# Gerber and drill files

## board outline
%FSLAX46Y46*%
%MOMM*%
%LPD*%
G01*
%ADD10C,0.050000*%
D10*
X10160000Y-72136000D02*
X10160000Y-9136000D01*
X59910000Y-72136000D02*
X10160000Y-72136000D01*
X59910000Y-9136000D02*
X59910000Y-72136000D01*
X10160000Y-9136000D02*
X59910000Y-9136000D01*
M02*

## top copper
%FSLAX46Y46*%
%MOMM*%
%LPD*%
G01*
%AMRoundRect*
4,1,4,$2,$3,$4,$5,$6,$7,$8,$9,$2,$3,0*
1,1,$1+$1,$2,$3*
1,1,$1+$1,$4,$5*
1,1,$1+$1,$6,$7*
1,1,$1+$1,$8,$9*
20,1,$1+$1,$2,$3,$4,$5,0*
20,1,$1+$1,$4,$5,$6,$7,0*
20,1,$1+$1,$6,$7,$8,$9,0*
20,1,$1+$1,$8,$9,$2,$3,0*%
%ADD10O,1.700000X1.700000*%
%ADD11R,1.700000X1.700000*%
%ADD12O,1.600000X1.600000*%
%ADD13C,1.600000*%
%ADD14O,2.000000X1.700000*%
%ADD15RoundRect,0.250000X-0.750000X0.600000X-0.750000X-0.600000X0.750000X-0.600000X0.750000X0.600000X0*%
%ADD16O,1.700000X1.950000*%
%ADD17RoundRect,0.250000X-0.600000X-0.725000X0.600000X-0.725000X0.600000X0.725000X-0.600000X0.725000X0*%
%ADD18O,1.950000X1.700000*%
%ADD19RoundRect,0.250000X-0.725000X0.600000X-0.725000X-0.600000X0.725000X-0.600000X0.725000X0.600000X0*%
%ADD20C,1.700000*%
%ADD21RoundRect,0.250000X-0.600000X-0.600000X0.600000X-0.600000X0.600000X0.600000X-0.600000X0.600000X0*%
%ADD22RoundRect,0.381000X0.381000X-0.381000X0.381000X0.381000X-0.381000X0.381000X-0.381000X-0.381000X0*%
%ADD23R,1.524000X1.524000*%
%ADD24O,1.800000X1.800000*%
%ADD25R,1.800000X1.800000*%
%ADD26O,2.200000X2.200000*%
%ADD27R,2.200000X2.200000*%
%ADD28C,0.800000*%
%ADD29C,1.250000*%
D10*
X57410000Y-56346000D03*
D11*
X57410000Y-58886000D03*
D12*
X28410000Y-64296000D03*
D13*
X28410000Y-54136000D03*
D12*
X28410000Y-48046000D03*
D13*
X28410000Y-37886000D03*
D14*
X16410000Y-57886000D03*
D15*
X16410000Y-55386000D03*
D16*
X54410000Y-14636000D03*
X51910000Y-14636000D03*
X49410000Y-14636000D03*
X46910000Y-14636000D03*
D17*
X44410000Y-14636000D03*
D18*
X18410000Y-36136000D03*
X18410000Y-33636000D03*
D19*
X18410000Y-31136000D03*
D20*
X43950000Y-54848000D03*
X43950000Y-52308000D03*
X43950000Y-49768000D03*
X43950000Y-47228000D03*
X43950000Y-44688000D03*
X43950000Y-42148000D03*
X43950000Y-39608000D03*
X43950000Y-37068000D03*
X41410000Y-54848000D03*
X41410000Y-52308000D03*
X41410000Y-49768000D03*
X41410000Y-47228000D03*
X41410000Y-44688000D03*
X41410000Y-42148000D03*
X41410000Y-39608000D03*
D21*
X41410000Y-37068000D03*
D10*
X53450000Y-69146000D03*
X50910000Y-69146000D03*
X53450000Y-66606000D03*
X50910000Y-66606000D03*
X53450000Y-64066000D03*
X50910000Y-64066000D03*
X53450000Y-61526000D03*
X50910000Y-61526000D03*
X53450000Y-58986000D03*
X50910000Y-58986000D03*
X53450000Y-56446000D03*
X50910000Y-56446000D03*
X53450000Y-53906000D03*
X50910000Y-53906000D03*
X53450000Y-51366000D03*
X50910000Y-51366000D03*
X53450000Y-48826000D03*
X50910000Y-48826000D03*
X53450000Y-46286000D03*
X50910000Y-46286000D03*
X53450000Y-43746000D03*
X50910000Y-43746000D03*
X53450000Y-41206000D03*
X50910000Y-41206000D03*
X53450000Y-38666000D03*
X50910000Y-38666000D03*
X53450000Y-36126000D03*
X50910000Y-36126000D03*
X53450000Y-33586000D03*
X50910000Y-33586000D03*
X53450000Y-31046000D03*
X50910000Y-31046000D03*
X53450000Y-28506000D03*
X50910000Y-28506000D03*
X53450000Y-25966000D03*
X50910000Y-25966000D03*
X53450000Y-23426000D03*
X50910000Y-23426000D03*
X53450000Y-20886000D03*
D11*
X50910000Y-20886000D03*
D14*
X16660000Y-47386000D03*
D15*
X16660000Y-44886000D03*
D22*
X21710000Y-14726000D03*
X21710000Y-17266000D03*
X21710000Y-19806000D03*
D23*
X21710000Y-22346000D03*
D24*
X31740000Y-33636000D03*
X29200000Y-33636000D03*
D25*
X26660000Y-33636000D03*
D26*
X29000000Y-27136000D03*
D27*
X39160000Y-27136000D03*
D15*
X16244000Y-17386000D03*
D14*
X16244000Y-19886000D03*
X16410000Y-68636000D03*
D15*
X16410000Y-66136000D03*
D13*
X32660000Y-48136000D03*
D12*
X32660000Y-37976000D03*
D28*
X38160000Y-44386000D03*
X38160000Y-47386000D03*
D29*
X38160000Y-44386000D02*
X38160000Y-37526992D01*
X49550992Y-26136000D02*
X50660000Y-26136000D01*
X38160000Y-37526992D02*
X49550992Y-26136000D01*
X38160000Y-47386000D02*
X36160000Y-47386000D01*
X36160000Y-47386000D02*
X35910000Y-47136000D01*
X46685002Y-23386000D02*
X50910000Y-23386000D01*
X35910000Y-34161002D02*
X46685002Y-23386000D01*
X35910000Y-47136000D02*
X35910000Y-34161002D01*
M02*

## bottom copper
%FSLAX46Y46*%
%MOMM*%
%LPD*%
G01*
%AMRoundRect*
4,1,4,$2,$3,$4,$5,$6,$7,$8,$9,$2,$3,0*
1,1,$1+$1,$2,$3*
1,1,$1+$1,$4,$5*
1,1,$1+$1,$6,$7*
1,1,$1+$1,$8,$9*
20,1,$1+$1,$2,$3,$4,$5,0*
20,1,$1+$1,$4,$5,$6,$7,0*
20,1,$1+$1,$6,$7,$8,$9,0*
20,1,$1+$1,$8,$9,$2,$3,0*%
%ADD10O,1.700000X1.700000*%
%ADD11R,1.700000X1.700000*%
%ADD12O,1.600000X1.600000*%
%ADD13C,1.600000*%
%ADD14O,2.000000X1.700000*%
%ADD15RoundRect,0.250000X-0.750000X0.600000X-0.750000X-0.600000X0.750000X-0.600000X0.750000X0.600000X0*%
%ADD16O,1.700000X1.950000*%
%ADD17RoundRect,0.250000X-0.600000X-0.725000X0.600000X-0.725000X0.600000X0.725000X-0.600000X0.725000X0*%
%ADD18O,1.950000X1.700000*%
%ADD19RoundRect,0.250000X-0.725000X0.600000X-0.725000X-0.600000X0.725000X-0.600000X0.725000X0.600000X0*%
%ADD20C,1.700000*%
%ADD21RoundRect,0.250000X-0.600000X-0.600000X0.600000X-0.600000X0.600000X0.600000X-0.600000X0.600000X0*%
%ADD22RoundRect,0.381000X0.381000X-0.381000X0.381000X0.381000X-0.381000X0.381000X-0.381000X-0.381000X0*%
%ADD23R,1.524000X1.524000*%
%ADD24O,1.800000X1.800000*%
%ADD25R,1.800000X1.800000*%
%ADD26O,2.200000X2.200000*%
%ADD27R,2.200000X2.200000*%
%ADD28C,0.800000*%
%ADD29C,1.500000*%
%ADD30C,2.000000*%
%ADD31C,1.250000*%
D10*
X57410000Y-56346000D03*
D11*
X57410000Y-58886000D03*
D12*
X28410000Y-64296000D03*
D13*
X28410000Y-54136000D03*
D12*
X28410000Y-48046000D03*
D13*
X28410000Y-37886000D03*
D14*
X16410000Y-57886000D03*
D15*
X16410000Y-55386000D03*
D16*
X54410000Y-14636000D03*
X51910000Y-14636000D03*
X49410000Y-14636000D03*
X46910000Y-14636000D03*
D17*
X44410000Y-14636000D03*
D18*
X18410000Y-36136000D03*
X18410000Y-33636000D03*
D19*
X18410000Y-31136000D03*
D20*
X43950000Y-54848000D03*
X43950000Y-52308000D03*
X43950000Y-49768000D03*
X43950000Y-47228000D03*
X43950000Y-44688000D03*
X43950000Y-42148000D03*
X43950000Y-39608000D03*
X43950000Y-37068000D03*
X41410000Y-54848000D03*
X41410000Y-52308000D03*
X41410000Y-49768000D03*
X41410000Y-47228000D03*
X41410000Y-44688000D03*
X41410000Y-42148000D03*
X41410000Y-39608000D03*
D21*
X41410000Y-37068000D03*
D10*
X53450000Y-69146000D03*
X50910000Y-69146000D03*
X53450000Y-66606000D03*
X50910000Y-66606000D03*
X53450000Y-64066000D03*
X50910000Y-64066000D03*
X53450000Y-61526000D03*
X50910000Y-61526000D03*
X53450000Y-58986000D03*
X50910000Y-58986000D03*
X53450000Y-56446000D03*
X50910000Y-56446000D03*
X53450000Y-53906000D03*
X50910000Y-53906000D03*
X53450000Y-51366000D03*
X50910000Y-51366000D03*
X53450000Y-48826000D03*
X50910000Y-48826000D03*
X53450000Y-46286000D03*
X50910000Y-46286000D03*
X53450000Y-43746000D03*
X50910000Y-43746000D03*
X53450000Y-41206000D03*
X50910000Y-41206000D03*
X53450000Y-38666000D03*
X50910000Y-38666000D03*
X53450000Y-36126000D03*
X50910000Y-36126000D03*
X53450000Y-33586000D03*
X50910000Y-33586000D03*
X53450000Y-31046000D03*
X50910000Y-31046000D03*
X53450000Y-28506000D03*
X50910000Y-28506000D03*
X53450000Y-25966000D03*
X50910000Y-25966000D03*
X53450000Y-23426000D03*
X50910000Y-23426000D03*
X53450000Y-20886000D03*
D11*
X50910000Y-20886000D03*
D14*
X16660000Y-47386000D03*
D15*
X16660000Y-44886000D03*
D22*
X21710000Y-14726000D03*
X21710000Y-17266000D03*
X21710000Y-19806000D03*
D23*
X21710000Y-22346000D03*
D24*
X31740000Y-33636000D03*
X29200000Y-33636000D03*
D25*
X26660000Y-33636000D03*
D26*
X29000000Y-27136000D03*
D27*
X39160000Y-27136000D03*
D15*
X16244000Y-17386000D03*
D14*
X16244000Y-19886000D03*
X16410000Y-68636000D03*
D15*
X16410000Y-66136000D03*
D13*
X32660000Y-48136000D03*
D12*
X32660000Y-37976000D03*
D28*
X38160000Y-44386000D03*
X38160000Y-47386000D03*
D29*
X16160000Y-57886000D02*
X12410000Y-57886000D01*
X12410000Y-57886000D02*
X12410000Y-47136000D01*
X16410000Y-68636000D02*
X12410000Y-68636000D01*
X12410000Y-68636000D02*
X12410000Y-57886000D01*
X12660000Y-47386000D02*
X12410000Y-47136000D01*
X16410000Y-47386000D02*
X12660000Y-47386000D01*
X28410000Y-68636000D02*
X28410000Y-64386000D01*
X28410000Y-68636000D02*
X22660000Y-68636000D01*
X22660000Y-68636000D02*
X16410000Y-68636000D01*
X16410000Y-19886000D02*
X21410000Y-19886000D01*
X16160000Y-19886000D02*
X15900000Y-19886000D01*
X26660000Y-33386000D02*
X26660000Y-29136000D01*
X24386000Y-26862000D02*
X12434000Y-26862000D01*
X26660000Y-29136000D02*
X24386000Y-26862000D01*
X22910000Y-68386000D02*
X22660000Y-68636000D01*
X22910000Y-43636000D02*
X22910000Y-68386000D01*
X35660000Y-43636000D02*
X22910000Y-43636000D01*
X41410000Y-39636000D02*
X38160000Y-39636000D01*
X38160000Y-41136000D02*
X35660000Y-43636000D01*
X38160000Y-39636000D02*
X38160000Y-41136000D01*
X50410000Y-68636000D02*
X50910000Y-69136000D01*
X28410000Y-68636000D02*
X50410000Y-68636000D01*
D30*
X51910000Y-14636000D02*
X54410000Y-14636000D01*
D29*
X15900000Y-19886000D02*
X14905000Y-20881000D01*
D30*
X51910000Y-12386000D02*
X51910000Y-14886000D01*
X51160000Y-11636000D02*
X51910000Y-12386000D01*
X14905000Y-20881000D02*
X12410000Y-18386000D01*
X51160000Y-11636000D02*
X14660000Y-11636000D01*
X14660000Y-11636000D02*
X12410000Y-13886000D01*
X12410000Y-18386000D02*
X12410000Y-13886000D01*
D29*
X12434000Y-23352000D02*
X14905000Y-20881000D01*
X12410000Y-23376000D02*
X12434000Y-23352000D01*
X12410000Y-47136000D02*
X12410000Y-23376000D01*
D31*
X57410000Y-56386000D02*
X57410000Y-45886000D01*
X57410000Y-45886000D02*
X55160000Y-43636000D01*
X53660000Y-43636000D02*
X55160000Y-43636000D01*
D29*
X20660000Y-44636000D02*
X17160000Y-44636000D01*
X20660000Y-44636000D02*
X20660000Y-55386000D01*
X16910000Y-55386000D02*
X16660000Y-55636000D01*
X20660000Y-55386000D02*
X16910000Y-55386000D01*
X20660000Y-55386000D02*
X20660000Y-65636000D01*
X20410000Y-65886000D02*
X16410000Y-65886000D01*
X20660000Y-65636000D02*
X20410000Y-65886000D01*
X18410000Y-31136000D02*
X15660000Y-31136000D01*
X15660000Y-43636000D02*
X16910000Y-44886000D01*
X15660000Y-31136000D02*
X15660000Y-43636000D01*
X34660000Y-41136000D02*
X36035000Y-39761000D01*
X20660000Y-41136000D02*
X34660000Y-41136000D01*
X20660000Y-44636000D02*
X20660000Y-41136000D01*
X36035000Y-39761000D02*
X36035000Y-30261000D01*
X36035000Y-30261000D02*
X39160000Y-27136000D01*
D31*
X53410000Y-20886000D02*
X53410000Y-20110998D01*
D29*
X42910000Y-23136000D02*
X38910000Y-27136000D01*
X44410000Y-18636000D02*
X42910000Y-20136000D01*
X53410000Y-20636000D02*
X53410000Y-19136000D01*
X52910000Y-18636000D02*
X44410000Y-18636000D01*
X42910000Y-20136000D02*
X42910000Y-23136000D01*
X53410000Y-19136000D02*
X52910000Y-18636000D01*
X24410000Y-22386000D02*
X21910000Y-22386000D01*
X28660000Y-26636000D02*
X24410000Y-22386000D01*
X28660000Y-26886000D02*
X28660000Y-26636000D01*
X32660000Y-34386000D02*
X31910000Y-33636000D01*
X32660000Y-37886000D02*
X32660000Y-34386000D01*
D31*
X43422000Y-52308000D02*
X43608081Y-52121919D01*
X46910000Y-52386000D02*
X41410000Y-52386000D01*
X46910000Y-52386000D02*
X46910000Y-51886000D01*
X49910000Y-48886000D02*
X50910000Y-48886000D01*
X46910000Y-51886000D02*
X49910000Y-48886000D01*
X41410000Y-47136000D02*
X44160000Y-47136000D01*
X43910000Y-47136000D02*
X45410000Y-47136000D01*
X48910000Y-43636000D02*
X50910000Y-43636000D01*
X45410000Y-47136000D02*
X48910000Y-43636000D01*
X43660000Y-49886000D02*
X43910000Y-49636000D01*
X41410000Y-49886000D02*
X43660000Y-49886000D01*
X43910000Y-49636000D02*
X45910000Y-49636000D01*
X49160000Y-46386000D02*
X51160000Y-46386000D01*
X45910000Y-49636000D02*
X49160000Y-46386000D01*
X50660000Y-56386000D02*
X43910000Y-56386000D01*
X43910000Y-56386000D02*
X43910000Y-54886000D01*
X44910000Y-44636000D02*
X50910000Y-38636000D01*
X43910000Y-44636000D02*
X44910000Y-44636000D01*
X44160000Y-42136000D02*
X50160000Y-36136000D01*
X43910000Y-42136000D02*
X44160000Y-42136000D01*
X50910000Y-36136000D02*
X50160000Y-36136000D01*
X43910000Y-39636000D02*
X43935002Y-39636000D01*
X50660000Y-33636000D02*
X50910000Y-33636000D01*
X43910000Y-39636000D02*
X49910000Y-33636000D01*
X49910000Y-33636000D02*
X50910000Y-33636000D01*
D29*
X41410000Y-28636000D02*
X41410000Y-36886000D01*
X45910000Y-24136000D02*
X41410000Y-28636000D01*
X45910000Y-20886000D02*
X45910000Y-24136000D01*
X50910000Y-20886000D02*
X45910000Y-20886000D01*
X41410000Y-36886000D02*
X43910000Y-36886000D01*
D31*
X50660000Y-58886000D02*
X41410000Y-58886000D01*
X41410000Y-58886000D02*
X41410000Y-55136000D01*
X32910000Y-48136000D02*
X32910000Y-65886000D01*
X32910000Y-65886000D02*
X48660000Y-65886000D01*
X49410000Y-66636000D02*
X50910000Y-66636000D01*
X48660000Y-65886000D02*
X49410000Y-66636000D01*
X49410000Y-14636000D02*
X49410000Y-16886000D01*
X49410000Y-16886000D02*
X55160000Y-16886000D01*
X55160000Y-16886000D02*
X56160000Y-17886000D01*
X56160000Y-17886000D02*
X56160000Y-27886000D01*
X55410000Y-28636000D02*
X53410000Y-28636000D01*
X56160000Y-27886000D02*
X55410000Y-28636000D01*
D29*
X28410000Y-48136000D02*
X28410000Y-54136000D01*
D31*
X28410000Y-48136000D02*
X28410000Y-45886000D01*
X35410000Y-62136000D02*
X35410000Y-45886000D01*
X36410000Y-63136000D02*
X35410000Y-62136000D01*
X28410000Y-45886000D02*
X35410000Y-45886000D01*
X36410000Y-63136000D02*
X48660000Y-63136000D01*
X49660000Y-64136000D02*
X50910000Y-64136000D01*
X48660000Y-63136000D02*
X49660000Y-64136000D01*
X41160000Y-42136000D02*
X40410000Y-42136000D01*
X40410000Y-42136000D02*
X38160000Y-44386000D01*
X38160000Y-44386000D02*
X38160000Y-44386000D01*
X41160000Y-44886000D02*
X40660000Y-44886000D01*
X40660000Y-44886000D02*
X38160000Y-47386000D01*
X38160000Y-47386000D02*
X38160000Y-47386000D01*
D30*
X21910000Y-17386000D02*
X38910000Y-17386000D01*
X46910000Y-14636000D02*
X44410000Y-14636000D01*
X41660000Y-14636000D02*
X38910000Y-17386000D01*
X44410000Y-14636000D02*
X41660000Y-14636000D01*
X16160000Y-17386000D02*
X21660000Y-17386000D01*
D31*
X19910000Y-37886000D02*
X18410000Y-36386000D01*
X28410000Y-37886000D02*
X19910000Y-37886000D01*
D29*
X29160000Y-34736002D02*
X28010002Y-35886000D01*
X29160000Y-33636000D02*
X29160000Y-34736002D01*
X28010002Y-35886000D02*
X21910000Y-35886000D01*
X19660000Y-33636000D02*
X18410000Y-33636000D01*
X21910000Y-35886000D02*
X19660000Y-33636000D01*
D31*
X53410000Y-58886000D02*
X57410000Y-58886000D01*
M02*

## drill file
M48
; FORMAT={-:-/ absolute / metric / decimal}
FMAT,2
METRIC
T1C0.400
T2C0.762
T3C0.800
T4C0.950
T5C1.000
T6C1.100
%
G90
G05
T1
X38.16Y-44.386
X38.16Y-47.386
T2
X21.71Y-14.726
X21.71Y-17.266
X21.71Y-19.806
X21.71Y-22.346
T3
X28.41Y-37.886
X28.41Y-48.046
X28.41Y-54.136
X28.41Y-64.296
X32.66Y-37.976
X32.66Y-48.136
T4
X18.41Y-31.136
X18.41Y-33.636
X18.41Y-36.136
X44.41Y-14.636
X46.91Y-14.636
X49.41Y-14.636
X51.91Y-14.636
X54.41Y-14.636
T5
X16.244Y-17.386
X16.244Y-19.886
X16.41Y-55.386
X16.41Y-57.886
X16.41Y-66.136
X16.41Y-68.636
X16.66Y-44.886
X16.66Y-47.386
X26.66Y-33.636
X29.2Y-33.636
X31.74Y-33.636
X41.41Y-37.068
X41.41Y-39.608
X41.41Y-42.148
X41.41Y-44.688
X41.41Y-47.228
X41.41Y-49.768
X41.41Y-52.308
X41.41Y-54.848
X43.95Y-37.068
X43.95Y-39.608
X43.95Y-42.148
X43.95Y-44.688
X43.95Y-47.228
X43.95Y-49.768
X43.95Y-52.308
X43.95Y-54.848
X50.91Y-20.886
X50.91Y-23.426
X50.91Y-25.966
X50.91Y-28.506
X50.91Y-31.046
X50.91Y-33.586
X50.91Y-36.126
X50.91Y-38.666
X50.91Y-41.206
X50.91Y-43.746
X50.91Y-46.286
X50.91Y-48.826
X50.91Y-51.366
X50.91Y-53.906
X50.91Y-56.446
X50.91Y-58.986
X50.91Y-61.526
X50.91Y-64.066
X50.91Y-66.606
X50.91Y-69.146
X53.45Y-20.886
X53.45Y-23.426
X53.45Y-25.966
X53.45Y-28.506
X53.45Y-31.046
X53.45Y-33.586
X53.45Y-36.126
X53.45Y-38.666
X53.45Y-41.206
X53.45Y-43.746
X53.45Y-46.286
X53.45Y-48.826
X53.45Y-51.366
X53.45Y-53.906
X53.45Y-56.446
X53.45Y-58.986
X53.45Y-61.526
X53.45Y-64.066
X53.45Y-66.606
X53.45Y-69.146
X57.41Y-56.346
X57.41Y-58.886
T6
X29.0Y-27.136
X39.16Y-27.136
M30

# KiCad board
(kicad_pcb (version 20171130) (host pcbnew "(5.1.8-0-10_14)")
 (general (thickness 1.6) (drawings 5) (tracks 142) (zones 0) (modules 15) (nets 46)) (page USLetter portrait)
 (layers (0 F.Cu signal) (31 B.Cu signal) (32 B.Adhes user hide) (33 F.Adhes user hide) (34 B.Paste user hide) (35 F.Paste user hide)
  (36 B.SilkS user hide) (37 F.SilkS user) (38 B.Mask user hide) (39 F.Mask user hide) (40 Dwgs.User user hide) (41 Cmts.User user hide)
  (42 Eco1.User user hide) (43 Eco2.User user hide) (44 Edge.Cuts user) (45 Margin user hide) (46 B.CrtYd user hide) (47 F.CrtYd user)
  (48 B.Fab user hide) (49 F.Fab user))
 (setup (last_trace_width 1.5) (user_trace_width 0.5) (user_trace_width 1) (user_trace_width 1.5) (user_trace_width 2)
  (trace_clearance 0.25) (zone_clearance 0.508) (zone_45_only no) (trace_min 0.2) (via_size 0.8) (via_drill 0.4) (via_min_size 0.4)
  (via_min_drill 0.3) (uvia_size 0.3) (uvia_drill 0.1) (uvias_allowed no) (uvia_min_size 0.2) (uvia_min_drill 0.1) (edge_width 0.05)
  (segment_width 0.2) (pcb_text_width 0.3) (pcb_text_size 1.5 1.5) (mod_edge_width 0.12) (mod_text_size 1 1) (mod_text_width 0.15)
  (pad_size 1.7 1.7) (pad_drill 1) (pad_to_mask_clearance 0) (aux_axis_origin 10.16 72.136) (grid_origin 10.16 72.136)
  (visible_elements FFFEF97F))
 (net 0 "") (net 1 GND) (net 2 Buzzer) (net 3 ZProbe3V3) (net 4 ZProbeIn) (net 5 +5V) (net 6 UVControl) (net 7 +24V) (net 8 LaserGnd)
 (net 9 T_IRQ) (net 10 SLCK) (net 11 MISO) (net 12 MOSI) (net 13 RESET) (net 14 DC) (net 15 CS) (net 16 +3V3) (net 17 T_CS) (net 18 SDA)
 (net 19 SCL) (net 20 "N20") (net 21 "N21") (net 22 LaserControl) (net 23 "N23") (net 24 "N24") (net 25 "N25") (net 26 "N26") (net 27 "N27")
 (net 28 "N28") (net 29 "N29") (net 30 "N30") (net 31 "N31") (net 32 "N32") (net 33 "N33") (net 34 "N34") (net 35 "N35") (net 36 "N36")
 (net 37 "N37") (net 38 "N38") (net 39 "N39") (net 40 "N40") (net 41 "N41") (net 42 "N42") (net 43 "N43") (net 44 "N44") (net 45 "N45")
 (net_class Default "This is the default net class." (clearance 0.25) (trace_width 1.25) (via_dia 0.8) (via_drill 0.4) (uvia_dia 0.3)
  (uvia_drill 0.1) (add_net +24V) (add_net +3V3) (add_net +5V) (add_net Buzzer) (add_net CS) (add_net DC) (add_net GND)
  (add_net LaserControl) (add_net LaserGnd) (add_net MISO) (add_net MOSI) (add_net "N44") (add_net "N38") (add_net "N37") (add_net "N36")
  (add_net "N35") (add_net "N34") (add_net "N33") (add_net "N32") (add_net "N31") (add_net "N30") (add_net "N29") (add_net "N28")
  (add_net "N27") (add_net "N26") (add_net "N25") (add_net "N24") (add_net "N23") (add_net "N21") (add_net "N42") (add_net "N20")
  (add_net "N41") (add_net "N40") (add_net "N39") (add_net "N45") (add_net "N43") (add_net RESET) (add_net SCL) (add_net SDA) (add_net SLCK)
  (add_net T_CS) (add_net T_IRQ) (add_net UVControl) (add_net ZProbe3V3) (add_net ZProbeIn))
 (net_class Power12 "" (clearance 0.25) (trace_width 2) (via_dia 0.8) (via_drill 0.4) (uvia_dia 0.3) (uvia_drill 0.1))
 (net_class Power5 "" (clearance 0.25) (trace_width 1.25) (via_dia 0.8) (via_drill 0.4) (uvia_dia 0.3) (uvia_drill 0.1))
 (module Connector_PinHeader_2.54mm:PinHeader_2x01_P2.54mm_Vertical (layer F.Cu) (at 57.41 58.886 90)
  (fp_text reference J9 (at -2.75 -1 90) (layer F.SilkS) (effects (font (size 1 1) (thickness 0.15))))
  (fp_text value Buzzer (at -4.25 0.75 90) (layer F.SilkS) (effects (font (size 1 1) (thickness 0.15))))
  (pad 2 thru_hole oval (at 2.54 0 90) (size 1.7 1.7) (drill 1) (layers *.Cu *.Mask) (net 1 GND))
  (pad 1 thru_hole rect (at 0 0 90) (size 1.7 1.7) (drill 1) (layers *.Cu *.Mask) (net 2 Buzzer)))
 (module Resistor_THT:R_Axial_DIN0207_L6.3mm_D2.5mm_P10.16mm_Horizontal (layer F.Cu) (at 28.41 54.136 270)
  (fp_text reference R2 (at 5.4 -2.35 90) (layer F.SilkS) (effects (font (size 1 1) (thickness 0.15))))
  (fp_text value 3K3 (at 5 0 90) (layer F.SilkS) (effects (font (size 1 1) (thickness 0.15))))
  (pad 2 thru_hole oval (at 10.16 0 270) (size 1.6 1.6) (drill 0.8) (layers *.Cu *.Mask) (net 1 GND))
  (pad 1 thru_hole circle (at 0 0 270) (size 1.6 1.6) (drill 0.8) (layers *.Cu *.Mask) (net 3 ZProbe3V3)))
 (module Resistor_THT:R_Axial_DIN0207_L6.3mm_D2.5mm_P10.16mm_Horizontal (layer F.Cu) (at 28.41 37.886 270)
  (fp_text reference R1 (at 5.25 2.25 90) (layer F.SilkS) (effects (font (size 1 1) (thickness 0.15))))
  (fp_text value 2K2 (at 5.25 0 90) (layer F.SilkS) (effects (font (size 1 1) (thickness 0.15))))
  (pad 2 thru_hole oval (at 10.16 0 270) (size 1.6 1.6) (drill 0.8) (layers *.Cu *.Mask) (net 3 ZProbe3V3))
  (pad 1 thru_hole circle (at 0 0 270) (size 1.6 1.6) (drill 0.8) (layers *.Cu *.Mask) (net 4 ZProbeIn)))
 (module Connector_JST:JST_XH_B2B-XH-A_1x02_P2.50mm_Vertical (layer F.Cu) (at 16.41 55.386 270)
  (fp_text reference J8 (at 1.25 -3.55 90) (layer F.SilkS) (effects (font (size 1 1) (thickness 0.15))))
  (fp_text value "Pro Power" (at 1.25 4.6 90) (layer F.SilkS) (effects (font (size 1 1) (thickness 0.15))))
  (pad 2 thru_hole oval (at 2.5 0 270) (size 1.7 2) (drill 1) (layers *.Cu *.Mask) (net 1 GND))
  (pad 1 thru_hole roundrect (at 0 0 270) (size 1.7 2) (drill 1) (layers *.Cu *.Mask) (roundrect_rratio 0.1470588235294118) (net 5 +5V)))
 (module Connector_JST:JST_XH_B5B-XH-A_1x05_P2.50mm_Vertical (layer F.Cu) (at 44.41 14.636)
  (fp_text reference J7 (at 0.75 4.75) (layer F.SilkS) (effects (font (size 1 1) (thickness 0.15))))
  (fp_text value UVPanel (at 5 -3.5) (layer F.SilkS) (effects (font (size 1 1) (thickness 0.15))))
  (pad 5 thru_hole oval (at 10 0) (size 1.7 1.95) (drill 0.95) (layers *.Cu *.Mask) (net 1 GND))
  (pad 4 thru_hole oval (at 7.5 0) (size 1.7 1.95) (drill 0.95) (layers *.Cu *.Mask) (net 1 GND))
  (pad 3 thru_hole oval (at 5 0) (size 1.7 1.95) (drill 0.95) (layers *.Cu *.Mask) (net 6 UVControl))
  (pad 2 thru_hole oval (at 2.5 0) (size 1.7 1.95) (drill 0.95) (layers *.Cu *.Mask) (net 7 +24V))
  (pad 1 thru_hole roundrect (at 0 0) (size 1.7 1.95) (drill 0.95) (layers *.Cu *.Mask) (roundrect_rratio 0.1470588235294118) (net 7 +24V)))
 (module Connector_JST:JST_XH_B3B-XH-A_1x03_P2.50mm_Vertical (layer F.Cu) (at 18.41 31.136 270)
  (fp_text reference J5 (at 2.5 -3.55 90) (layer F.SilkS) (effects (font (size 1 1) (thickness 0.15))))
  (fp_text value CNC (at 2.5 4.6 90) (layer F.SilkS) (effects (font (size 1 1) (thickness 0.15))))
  (pad 3 thru_hole oval (at 5 0 270) (size 1.7 1.95) (drill 0.95) (layers *.Cu *.Mask) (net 4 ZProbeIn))
  (pad 2 thru_hole oval (at 2.5 0 270) (size 1.7 1.95) (drill 0.95) (layers *.Cu *.Mask) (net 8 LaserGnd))
  (pad 1 thru_hole roundrect (at 0 0 270) (size 1.7 1.95) (drill 0.95) (layers *.Cu *.Mask) (roundrect_rratio 0.1470588235294118)
   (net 5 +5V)))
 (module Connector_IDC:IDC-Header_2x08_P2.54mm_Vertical (layer F.Cu) (at 41.41 37.068)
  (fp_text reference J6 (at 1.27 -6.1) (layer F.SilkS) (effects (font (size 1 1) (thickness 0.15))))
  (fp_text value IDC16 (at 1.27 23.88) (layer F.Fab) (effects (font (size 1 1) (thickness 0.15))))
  (pad 16 thru_hole circle (at 2.54 17.78) (size 1.7 1.7) (drill 1) (layers *.Cu *.Mask) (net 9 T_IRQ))
  (pad 14 thru_hole circle (at 2.54 15.24) (size 1.7 1.7) (drill 1) (layers *.Cu *.Mask) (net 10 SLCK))
  (pad 12 thru_hole circle (at 2.54 12.7) (size 1.7 1.7) (drill 1) (layers *.Cu *.Mask) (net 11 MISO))
  (pad 10 thru_hole circle (at 2.54 10.16) (size 1.7 1.7) (drill 1) (layers *.Cu *.Mask) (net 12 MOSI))
  (pad 8 thru_hole circle (at 2.54 7.62) (size 1.7 1.7) (drill 1) (layers *.Cu *.Mask) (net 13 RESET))
  (pad 6 thru_hole circle (at 2.54 5.08) (size 1.7 1.7) (drill 1) (layers *.Cu *.Mask) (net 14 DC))
  (pad 4 thru_hole circle (at 2.54 2.54) (size 1.7 1.7) (drill 1) (layers *.Cu *.Mask) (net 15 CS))
  (pad 2 thru_hole circle (at 2.54 0) (size 1.7 1.7) (drill 1) (layers *.Cu *.Mask) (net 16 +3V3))
  (pad 15 thru_hole circle (at 0 17.78) (size 1.7 1.7) (drill 1) (layers *.Cu *.Mask) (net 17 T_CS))
  (pad 13 thru_hole circle (at 0 15.24) (size 1.7 1.7) (drill 1) (layers *.Cu *.Mask) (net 10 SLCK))
  (pad 11 thru_hole circle (at 0 12.7) (size 1.7 1.7) (drill 1) (layers *.Cu *.Mask) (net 11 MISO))
  (pad 9 thru_hole circle (at 0 10.16) (size 1.7 1.7) (drill 1) (layers *.Cu *.Mask) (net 12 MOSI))
  (pad 7 thru_hole circle (at 0 7.62) (size 1.7 1.7) (drill 1) (layers *.Cu *.Mask) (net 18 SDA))
  (pad 5 thru_hole circle (at 0 5.08) (size 1.7 1.7) (drill 1) (layers *.Cu *.Mask) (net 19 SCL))
  (pad 3 thru_hole circle (at 0 2.54) (size 1.7 1.7) (drill 1) (layers *.Cu *.Mask) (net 1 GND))
  (pad 1 thru_hole roundrect (at 0 0) (size 1.7 1.7) (drill 1) (layers *.Cu *.Mask) (roundrect_rratio 0.1470588235294118) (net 16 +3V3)))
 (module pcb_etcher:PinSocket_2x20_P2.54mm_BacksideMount (layer F.Cu) (at 50.91 20.886)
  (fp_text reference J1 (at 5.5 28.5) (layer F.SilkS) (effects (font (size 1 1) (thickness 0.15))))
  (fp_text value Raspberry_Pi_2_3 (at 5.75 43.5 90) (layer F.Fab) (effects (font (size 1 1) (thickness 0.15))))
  (pad 40 thru_hole oval (at 2.54 48.26) (size 1.7 1.7) (drill 1) (layers *.Cu *.Mask) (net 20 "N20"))
  (pad 39 thru_hole oval (at 0 48.26) (size 1.7 1.7) (drill 1) (layers *.Cu *.Mask) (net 1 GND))
  (pad 38 thru_hole oval (at 2.54 45.72) (size 1.7 1.7) (drill 1) (layers *.Cu *.Mask) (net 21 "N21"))
  (pad 37 thru_hole oval (at 0 45.72) (size 1.7 1.7) (drill 1) (layers *.Cu *.Mask) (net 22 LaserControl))
  (pad 36 thru_hole oval (at 2.54 43.18) (size 1.7 1.7) (drill 1) (layers *.Cu *.Mask) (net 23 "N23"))
  (pad 35 thru_hole oval (at 0 43.18) (size 1.7 1.7) (drill 1) (layers *.Cu *.Mask) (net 3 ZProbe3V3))
  (pad 34 thru_hole oval (at 2.54 40.64) (size 1.7 1.7) (drill 1) (layers *.Cu *.Mask) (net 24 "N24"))
  (pad 33 thru_hole oval (at 0 40.64) (size 1.7 1.7) (drill 1) (layers *.Cu *.Mask) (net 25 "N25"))
  (pad 32 thru_hole oval (at 2.54 38.1) (size 1.7 1.7) (drill 1) (layers *.Cu *.Mask) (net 2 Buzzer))
  (pad 31 thru_hole oval (at 0 38.1) (size 1.7 1.7) (drill 1) (layers *.Cu *.Mask) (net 17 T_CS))
  (pad 30 thru_hole oval (at 2.54 35.56) (size 1.7 1.7) (drill 1) (layers *.Cu *.Mask) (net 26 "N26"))
  (pad 29 thru_hole oval (at 0 35.56) (size 1.7 1.7) (drill 1) (layers *.Cu *.Mask) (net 9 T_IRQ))
  (pad 28 thru_hole oval (at 2.54 33.02) (size 1.7 1.7) (drill 1) (layers *.Cu *.Mask) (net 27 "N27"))
  (pad 27 thru_hole oval (at 0 33.02) (size 1.7 1.7) (drill 1) (layers *.Cu *.Mask) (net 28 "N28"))
  (pad 26 thru_hole oval (at 2.54 30.48) (size 1.7 1.7) (drill 1) (layers *.Cu *.Mask) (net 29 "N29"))
  (pad 25 thru_hole oval (at 0 30.48) (size 1.7 1.7) (drill 1) (layers *.Cu *.Mask) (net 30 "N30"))
  (pad 24 thru_hole oval (at 2.54 27.94) (size 1.7 1.7) (drill 1) (layers *.Cu *.Mask) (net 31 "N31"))
  (pad 23 thru_hole oval (at 0 27.94) (size 1.7 1.7) (drill 1) (layers *.Cu *.Mask) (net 10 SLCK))
  (pad 22 thru_hole oval (at 2.54 25.4) (size 1.7 1.7) (drill 1) (layers *.Cu *.Mask) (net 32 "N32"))
  (pad 21 thru_hole oval (at 0 25.4) (size 1.7 1.7) (drill 1) (layers *.Cu *.Mask) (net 11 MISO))
  (pad 20 thru_hole oval (at 2.54 22.86) (size 1.7 1.7) (drill 1) (layers *.Cu *.Mask) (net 1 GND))
  (pad 19 thru_hole oval (at 0 22.86) (size 1.7 1.7) (drill 1) (layers *.Cu *.Mask) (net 12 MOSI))
  (pad 18 thru_hole oval (at 2.54 20.32) (size 1.7 1.7) (drill 1) (layers *.Cu *.Mask) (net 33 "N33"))
  (pad 17 thru_hole oval (at 0 20.32) (size 1.7 1.7) (drill 1) (layers *.Cu *.Mask) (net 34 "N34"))
  (pad 16 thru_hole oval (at 2.54 17.78) (size 1.7 1.7) (drill 1) (layers *.Cu *.Mask) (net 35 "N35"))
  (pad 15 thru_hole oval (at 0 17.78) (size 1.7 1.7) (drill 1) (layers *.Cu *.Mask) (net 13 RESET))
  (pad 14 thru_hole oval (at 2.54 15.24) (size 1.7 1.7) (drill 1) (layers *.Cu *.Mask) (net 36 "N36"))
  (pad 13 thru_hole oval (at 0 15.24) (size 1.7 1.7) (drill 1) (layers *.Cu *.Mask) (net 14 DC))
  (pad 12 thru_hole oval (at 2.54 12.7) (size 1.7 1.7) (drill 1) (layers *.Cu *.Mask) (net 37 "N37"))
  (pad 11 thru_hole oval (at 0 12.7) (size 1.7 1.7) (drill 1) (layers *.Cu *.Mask) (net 15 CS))
  (pad 10 thru_hole oval (at 2.54 10.16) (size 1.7 1.7) (drill 1) (layers *.Cu *.Mask) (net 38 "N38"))
  (pad 9 thru_hole oval (at 0 10.16) (size 1.7 1.7) (drill 1) (layers *.Cu *.Mask) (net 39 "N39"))
  (pad 8 thru_hole oval (at 2.54 7.62) (size 1.7 1.7) (drill 1) (layers *.Cu *.Mask) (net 6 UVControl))
  (pad 7 thru_hole oval (at 0 7.62) (size 1.7 1.7) (drill 1) (layers *.Cu *.Mask) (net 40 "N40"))
  (pad 6 thru_hole oval (at 2.54 5.08) (size 1.7 1.7) (drill 1) (layers *.Cu *.Mask) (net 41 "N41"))
  (pad 5 thru_hole oval (at 0 5.08) (size 1.7 1.7) (drill 1) (layers *.Cu *.Mask) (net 19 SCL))
  (pad 4 thru_hole oval (at 2.54 2.54) (size 1.7 1.7) (drill 1) (layers *.Cu *.Mask) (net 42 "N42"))
  (pad 3 thru_hole oval (at 0 2.54) (size 1.7 1.7) (drill 1) (layers *.Cu *.Mask) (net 18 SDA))
  (pad 2 thru_hole oval (at 2.54 0) (size 1.7 1.7) (drill 1) (layers *.Cu *.Mask) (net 5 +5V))
  (pad 1 thru_hole rect (at 0 0) (size 1.7 1.7) (drill 1) (layers *.Cu *.Mask) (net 16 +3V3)))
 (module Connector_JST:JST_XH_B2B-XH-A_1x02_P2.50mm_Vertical (layer F.Cu) (at 16.66 44.886 270)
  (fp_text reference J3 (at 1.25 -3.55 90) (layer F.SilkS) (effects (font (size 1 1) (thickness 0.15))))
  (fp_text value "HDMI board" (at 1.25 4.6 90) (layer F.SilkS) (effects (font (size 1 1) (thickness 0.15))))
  (pad 2 thru_hole oval (at 2.5 0 270) (size 1.7 2) (drill 1) (layers *.Cu *.Mask) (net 1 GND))
  (pad 1 thru_hole roundrect (at 0 0 270) (size 1.7 2) (drill 1) (layers *.Cu *.Mask) (roundrect_rratio 0.1470588235294118) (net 5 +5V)))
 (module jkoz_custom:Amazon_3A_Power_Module (layer F.Cu) (at 29.66 18.636 90)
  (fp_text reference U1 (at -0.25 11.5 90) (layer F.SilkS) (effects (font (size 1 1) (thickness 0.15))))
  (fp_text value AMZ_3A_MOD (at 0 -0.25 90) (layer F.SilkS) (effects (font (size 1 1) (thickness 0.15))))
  (pad 4 thru_hole roundrect (at 3.91 -7.95 90) (size 1.524 1.524) (drill 0.762) (layers *.Cu *.Mask) (roundrect_rratio 0.25) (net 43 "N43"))
  (pad 3 thru_hole roundrect (at 1.37 -7.95 90) (size 1.524 1.524) (drill 0.762) (layers *.Cu *.Mask) (roundrect_rratio 0.25) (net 7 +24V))
  (pad 2 thru_hole roundrect (at -1.17 -7.95 90) (size 1.524 1.524) (drill 0.762) (layers *.Cu *.Mask) (roundrect_rratio 0.25) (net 1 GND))
  (pad 1 thru_hole rect (at -3.71 -7.95 90) (size 1.524 1.524) (drill 0.762) (layers *.Cu *.Mask) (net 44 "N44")))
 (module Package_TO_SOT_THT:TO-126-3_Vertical (layer F.Cu) (at 26.66 33.636)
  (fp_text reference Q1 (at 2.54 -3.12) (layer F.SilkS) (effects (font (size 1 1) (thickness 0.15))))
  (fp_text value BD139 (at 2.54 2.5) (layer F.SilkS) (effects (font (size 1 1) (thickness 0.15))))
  (pad 3 thru_hole oval (at 5.08 0) (size 1.8 1.8) (drill 1) (layers *.Cu *.Mask) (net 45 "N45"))
  (pad 2 thru_hole oval (at 2.54 0) (size 1.8 1.8) (drill 1) (layers *.Cu *.Mask) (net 8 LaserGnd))
  (pad 1 thru_hole rect (at 0 0) (size 1.8 1.8) (drill 1) (layers *.Cu *.Mask) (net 1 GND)))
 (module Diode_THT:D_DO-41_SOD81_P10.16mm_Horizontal (layer F.Cu) (at 39.16 27.136 180)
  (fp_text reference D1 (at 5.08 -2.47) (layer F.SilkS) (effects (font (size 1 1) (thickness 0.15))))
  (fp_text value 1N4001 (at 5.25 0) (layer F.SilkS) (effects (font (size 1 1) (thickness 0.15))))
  (pad 2 thru_hole oval (at 10.16 0 180) (size 2.2 2.2) (drill 1.1) (layers *.Cu *.Mask) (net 44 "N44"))
  (pad 1 thru_hole rect (at 0 0 180) (size 2.2 2.2) (drill 1.1) (layers *.Cu *.Mask) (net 5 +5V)))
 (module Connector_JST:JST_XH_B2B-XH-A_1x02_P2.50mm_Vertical (layer F.Cu) (at 16.244 17.386 270)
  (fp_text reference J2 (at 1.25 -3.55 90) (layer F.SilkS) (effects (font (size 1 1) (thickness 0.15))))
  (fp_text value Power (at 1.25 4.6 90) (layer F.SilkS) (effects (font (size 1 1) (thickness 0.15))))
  (pad 1 thru_hole roundrect (at 0 0 270) (size 1.7 2) (drill 1) (layers *.Cu *.Mask) (roundrect_rratio 0.1470588235294118) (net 7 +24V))
  (pad 2 thru_hole oval (at 2.5 0 270) (size 1.7 2) (drill 1) (layers *.Cu *.Mask) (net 1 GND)))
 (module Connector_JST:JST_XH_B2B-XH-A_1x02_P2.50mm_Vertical (layer F.Cu) (at 16.41 66.136 270)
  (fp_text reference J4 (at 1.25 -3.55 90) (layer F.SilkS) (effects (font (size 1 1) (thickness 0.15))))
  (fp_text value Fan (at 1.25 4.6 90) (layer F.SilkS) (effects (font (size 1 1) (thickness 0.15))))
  (pad 2 thru_hole oval (at 2.5 0 270) (size 1.7 2) (drill 1) (layers *.Cu *.Mask) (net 1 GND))
  (pad 1 thru_hole roundrect (at 0 0 270) (size 1.7 2) (drill 1) (layers *.Cu *.Mask) (roundrect_rratio 0.1470588235294118) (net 5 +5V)))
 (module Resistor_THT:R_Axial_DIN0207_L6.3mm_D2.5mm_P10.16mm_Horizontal (layer F.Cu) (at 32.66 48.136 90)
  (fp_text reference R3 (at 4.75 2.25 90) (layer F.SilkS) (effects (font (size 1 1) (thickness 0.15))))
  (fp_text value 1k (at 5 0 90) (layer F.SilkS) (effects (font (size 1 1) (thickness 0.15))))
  (pad 1 thru_hole circle (at 0 0 90) (size 1.6 1.6) (drill 0.8) (layers *.Cu *.Mask) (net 22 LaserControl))
  (pad 2 thru_hole oval (at 10.16 0 90) (size 1.6 1.6) (drill 0.8) (layers *.Cu *.Mask) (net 45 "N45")))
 (gr_line (start 10.16 72.136) (end 10.16 9.136) (layer Edge.Cuts) (width 0.05))
 (gr_line (start 59.91 72.136) (end 10.16 72.136) (layer Edge.Cuts) (width 0.05))
 (gr_line (start 59.91 9.136) (end 59.91 72.136) (layer Edge.Cuts) (width 0.05))
 (gr_line (start 10.16 9.136) (end 59.91 9.136) (layer Edge.Cuts) (width 0.05))
 (segment (start 16.16 57.886) (end 12.41 57.886) (width 1.5) (layer B.Cu) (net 1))
 (segment (start 12.41 57.886) (end 12.41 47.136) (width 1.5) (layer B.Cu) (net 1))
 (segment (start 16.41 68.636) (end 12.41 68.636) (width 1.5) (layer B.Cu) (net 1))
 (segment (start 12.41 68.636) (end 12.41 57.886) (width 1.5) (layer B.Cu) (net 1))
 (segment (start 12.66 47.386) (end 12.41 47.136) (width 1.5) (layer B.Cu) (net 1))
 (segment (start 16.41 47.386) (end 12.66 47.386) (width 1.5) (layer B.Cu) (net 1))
 (segment (start 28.41 68.636) (end 28.41 64.386) (width 1.5) (layer B.Cu) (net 1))
 (segment (start 28.41 68.636) (end 22.66 68.636) (width 1.5) (layer B.Cu) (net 1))
 (segment (start 22.66 68.636) (end 16.41 68.636) (width 1.5) (layer B.Cu) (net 1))
 (segment (start 16.41 19.886) (end 21.41 19.886) (width 1.5) (layer B.Cu) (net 1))
 (segment (start 16.16 19.886) (end 15.9 19.886) (width 1.5) (layer B.Cu) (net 1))
 (segment (start 26.66 33.386) (end 26.66 29.136) (width 1.5) (layer B.Cu) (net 1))
 (segment (start 24.386 26.862) (end 12.434 26.862) (width 1.5) (layer B.Cu) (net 1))
 (segment (start 26.66 29.136) (end 24.386 26.862) (width 1.5) (layer B.Cu) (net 1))
 (segment (start 22.91 68.386) (end 22.66 68.636) (width 1.5) (layer B.Cu) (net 1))
 (segment (start 22.91 43.636) (end 22.91 68.386) (width 1.5) (layer B.Cu) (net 1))
 (segment (start 35.66 43.636) (end 22.91 43.636) (width 1.5) (layer B.Cu) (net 1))
 (segment (start 41.41 39.636) (end 38.16 39.636) (width 1.5) (layer B.Cu) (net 1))
 (segment (start 38.16 41.136) (end 35.66 43.636) (width 1.5) (layer B.Cu) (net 1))
 (segment (start 38.16 39.636) (end 38.16 41.136) (width 1.5) (layer B.Cu) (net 1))
 (segment (start 50.41 68.636) (end 50.91 69.136) (width 1.5) (layer B.Cu) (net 1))
 (segment (start 28.41 68.636) (end 50.41 68.636) (width 1.5) (layer B.Cu) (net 1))
 (segment (start 51.91 14.636) (end 54.41 14.636) (width 2) (layer B.Cu) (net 1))
 (segment (start 15.9 19.886) (end 14.905 20.881) (width 1.5) (layer B.Cu) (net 1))
 (segment (start 51.91 12.386) (end 51.91 14.886) (width 2) (layer B.Cu) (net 1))
 (segment (start 51.16 11.636) (end 51.91 12.386) (width 2) (layer B.Cu) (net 1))
 (segment (start 14.905 20.881) (end 12.41 18.386) (width 2) (layer B.Cu) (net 1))
 (segment (start 51.16 11.636) (end 14.66 11.636) (width 2) (layer B.Cu) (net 1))
 (segment (start 14.66 11.636) (end 12.41 13.886) (width 2) (layer B.Cu) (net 1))
 (segment (start 12.41 18.386) (end 12.41 13.886) (width 2) (layer B.Cu) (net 1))
 (segment (start 12.434 23.352) (end 14.905 20.881) (width 1.5) (layer B.Cu) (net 1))
 (segment (start 12.41 23.376) (end 12.434 23.352) (width 1.5) (layer B.Cu) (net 1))
 (segment (start 12.41 47.136) (end 12.41 23.376) (width 1.5) (layer B.Cu) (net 1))
 (segment (start 57.41 56.386) (end 57.41 45.886) (width 1.25) (layer B.Cu) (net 1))
 (segment (start 57.41 45.886) (end 55.16 43.636) (width 1.25) (layer B.Cu) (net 1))
 (segment (start 53.66 43.636) (end 55.16 43.636) (width 1.25) (layer B.Cu) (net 1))
 (segment (start 20.66 44.636) (end 17.16 44.636) (width 1.5) (layer B.Cu) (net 5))
 (segment (start 20.66 44.636) (end 20.66 55.386) (width 1.5) (layer B.Cu) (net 5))
 (segment (start 16.91 55.386) (end 16.66 55.636) (width 1.5) (layer B.Cu) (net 5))
 (segment (start 20.66 55.386) (end 16.91 55.386) (width 1.5) (layer B.Cu) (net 5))
 (segment (start 20.66 55.386) (end 20.66 65.636) (width 1.5) (layer B.Cu) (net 5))
 (segment (start 20.41 65.886) (end 16.41 65.886) (width 1.5) (layer B.Cu) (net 5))
 (segment (start 20.66 65.636) (end 20.41 65.886) (width 1.5) (layer B.Cu) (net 5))
 (segment (start 18.41 31.136) (end 15.66 31.136) (width 1.5) (layer B.Cu) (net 5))
 (segment (start 15.66 43.636) (end 16.91 44.886) (width 1.5) (layer B.Cu) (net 5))
 (segment (start 15.66 31.136) (end 15.66 43.636) (width 1.5) (layer B.Cu) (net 5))
 (segment (start 34.66 41.136) (end 36.035 39.761) (width 1.5) (layer B.Cu) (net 5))
 (segment (start 20.66 41.136) (end 34.66 41.136) (width 1.5) (layer B.Cu) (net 5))
 (segment (start 20.66 44.636) (end 20.66 41.136) (width 1.5) (layer B.Cu) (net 5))
 (segment (start 36.035 39.761) (end 36.035 30.261) (width 1.5) (layer B.Cu) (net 5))
 (segment (start 36.035 30.261) (end 39.16 27.136) (width 1.5) (layer B.Cu) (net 5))
 (segment (start 53.41 20.886) (end 53.41 20.110998) (width 1.25) (layer B.Cu) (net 5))
 (segment (start 42.91 23.136) (end 38.91 27.136) (width 1.5) (layer B.Cu) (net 5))
 (segment (start 44.41 18.636) (end 42.91 20.136) (width 1.5) (layer B.Cu) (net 5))
 (segment (start 53.41 20.636) (end 53.41 19.136) (width 1.5) (layer B.Cu) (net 5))
 (segment (start 52.91 18.636) (end 44.41 18.636) (width 1.5) (layer B.Cu) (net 5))
 (segment (start 42.91 20.136) (end 42.91 23.136) (width 1.5) (layer B.Cu) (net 5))
 (segment (start 53.41 19.136) (end 52.91 18.636) (width 1.5) (layer B.Cu) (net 5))
 (segment (start 24.41 22.386) (end 21.91 22.386) (width 1.5) (layer B.Cu) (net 44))
 (segment (start 28.66 26.636) (end 24.41 22.386) (width 1.5) (layer B.Cu) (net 44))
 (segment (start 28.66 26.886) (end 28.66 26.636) (width 1.5) (layer B.Cu) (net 44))
 (segment (start 32.66 34.386) (end 31.91 33.636) (width 1.5) (layer B.Cu) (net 45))
 (segment (start 32.66 37.886) (end 32.66 34.386) (width 1.5) (layer B.Cu) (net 45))
 (segment (start 43.422 52.308) (end 43.608081 52.121919) (width 1.25) (layer B.Cu) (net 10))
 (segment (start 46.91 52.386) (end 41.41 52.386) (width 1.25) (layer B.Cu) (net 10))
 (segment (start 46.91 52.386) (end 46.91 51.886) (width 1.25) (layer B.Cu) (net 10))
 (segment (start 49.91 48.886) (end 50.91 48.886) (width 1.25) (layer B.Cu) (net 10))
 (segment (start 46.91 51.886) (end 49.91 48.886) (width 1.25) (layer B.Cu) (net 10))
 (segment (start 41.41 47.136) (end 44.16 47.136) (width 1.25) (layer B.Cu) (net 12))
 (segment (start 43.91 47.136) (end 45.41 47.136) (width 1.25) (layer B.Cu) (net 12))
 (segment (start 48.91 43.636) (end 50.91 43.636) (width 1.25) (layer B.Cu) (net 12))
 (segment (start 45.41 47.136) (end 48.91 43.636) (width 1.25) (layer B.Cu) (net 12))
 (segment (start 43.66 49.886) (end 43.91 49.636) (width 1.25) (layer B.Cu) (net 11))
 (segment (start 41.41 49.886) (end 43.66 49.886) (width 1.25) (layer B.Cu) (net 11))
 (segment (start 43.91 49.636) (end 45.91 49.636) (width 1.25) (layer B.Cu) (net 11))
 (segment (start 49.16 46.386) (end 51.16 46.386) (width 1.25) (layer B.Cu) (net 11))
 (segment (start 45.91 49.636) (end 49.16 46.386) (width 1.25) (layer B.Cu) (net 11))
 (segment (start 50.66 56.386) (end 43.91 56.386) (width 1.25) (layer B.Cu) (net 9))
 (segment (start 43.91 56.386) (end 43.91 54.886) (width 1.25) (layer B.Cu) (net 9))
 (segment (start 44.91 44.636) (end 50.91 38.636) (width 1.25) (layer B.Cu) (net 13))
 (segment (start 43.91 44.636) (end 44.91 44.636) (width 1.25) (layer B.Cu) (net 13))
 (segment (start 44.16 42.136) (end 50.16 36.136) (width 1.25) (layer B.Cu) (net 14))
 (segment (start 43.91 42.136) (end 44.16 42.136) (width 1.25) (layer B.Cu) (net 14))
 (segment (start 50.91 36.136) (end 50.16 36.136) (width 1.25) (layer B.Cu) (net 14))
 (segment (start 43.91 39.636) (end 43.935002 39.636) (width 1.25) (layer B.Cu) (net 15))
 (segment (start 50.66 33.636) (end 50.91 33.636) (width 1.25) (layer B.Cu) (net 15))
 (segment (start 43.91 39.636) (end 49.91 33.636) (width 1.25) (layer B.Cu) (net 15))
 (segment (start 49.91 33.636) (end 50.91 33.636) (width 1.25) (layer B.Cu) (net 15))
 (segment (start 41.41 28.636) (end 41.41 36.886) (width 1.5) (layer B.Cu) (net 16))
 (segment (start 45.91 24.136) (end 41.41 28.636) (width 1.5) (layer B.Cu) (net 16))
 (segment (start 45.91 20.886) (end 45.91 24.136) (width 1.5) (layer B.Cu) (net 16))
 (segment (start 50.91 20.886) (end 45.91 20.886) (width 1.5) (layer B.Cu) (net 16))
 (segment (start 41.41 36.886) (end 43.91 36.886) (width 1.5) (layer B.Cu) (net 16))
 (segment (start 50.66 58.886) (end 41.41 58.886) (width 1.25) (layer B.Cu) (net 17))
 (segment (start 41.41 58.886) (end 41.41 55.136) (width 1.25) (layer B.Cu) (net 17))
 (segment (start 32.91 48.136) (end 32.91 65.886) (width 1.25) (layer B.Cu) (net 22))
 (segment (start 32.91 65.886) (end 48.66 65.886) (width 1.25) (layer B.Cu) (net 22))
 (segment (start 49.41 66.636) (end 50.91 66.636) (width 1.25) (layer B.Cu) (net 22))
 (segment (start 48.66 65.886) (end 49.41 66.636) (width 1.25) (layer B.Cu) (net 22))
 (segment (start 49.41 14.636) (end 49.41 16.886) (width 1.25) (layer B.Cu) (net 6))
 (segment (start 49.41 16.886) (end 55.16 16.886) (width 1.25) (layer B.Cu) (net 6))
 (segment (start 55.16 16.886) (end 56.16 17.886) (width 1.25) (layer B.Cu) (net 6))
 (segment (start 56.16 17.886) (end 56.16 27.886) (width 1.25) (layer B.Cu) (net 6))
 (segment (start 55.41 28.636) (end 53.41 28.636) (width 1.25) (layer B.Cu) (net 6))
 (segment (start 56.16 27.886) (end 55.41 28.636) (width 1.25) (layer B.Cu) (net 6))
 (segment (start 28.41 48.136) (end 28.41 54.136) (width 1.5) (layer B.Cu) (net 3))
 (segment (start 28.41 48.136) (end 28.41 45.886) (width 1.25) (layer B.Cu) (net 3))
 (segment (start 35.41 62.136) (end 35.41 45.886) (width 1.25) (layer B.Cu) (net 3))
 (segment (start 36.41 63.136) (end 35.41 62.136) (width 1.25) (layer B.Cu) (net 3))
 (segment (start 28.41 45.886) (end 35.41 45.886) (width 1.25) (layer B.Cu) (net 3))
 (segment (start 36.41 63.136) (end 48.66 63.136) (width 1.25) (layer B.Cu) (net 3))
 (segment (start 49.66 64.136) (end 50.91 64.136) (width 1.25) (layer B.Cu) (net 3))
 (segment (start 48.66 63.136) (end 49.66 64.136) (width 1.25) (layer B.Cu) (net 3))
 (segment (start 41.16 42.136) (end 40.41 42.136) (width 1.25) (layer B.Cu) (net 19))
 (segment (start 40.41 42.136) (end 38.16 44.386) (width 1.25) (layer B.Cu) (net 19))
 (segment (start 38.16 44.386) (end 38.16 44.386) (width 1.25) (layer B.Cu) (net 19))
 (via (at 38.16 44.386) (size 0.8) (drill 0.4) (layers F.Cu B.Cu) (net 19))
 (segment (start 38.16 44.386) (end 38.16 37.526992) (width 1.25) (layer F.Cu) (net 19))
 (segment (start 49.550992 26.136) (end 50.66 26.136) (width 1.25) (layer F.Cu) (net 19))
 (segment (start 38.16 37.526992) (end 49.550992 26.136) (width 1.25) (layer F.Cu) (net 19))
 (segment (start 41.16 44.886) (end 40.66 44.886) (width 1.25) (layer B.Cu) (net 18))
 (segment (start 40.66 44.886) (end 38.16 47.386) (width 1.25) (layer B.Cu) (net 18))
 (segment (start 38.16 47.386) (end 38.16 47.386) (width 1.25) (layer B.Cu) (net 18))
 (via (at 38.16 47.386) (size 0.8) (drill 0.4) (layers F.Cu B.Cu) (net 18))
 (segment (start 38.16 47.386) (end 36.16 47.386) (width 1.25) (layer F.Cu) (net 18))
 (segment (start 36.16 47.386) (end 35.91 47.136) (width 1.25) (layer F.Cu) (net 18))
 (segment (start 46.685002 23.386) (end 50.91 23.386) (width 1.25) (layer F.Cu) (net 18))
 (segment (start 35.91 34.161002) (end 46.685002 23.386) (width 1.25) (layer F.Cu) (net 18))
 (segment (start 35.91 47.136) (end 35.91 34.161002) (width 1.25) (layer F.Cu) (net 18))
 (segment (start 21.91 17.386) (end 38.91 17.386) (width 2) (layer B.Cu) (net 7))
 (segment (start 46.91 14.636) (end 44.41 14.636) (width 2) (layer B.Cu) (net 7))
 (segment (start 41.66 14.636) (end 38.91 17.386) (width 2) (layer B.Cu) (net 7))
 (segment (start 44.41 14.636) (end 41.66 14.636) (width 2) (layer B.Cu) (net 7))
 (segment (start 16.16 17.386) (end 21.66 17.386) (width 2) (layer B.Cu) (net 7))
 (segment (start 19.91 37.886) (end 18.41 36.386) (width 1.25) (layer B.Cu) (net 4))
 (segment (start 28.41 37.886) (end 19.91 37.886) (width 1.25) (layer B.Cu) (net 4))
 (segment (start 29.16 34.736002) (end 28.010002 35.886) (width 1.5) (layer B.Cu) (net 8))
 (segment (start 29.16 33.636) (end 29.16 34.736002) (width 1.5) (layer B.Cu) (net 8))
 (segment (start 28.010002 35.886) (end 21.91 35.886) (width 1.5) (layer B.Cu) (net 8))
 (segment (start 19.66 33.636) (end 18.41 33.636) (width 1.5) (layer B.Cu) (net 8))
 (segment (start 21.91 35.886) (end 19.66 33.636) (width 1.5) (layer B.Cu) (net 8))
 (segment (start 53.41 58.886) (end 57.41 58.886) (width 1.25) (layer B.Cu) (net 2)))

